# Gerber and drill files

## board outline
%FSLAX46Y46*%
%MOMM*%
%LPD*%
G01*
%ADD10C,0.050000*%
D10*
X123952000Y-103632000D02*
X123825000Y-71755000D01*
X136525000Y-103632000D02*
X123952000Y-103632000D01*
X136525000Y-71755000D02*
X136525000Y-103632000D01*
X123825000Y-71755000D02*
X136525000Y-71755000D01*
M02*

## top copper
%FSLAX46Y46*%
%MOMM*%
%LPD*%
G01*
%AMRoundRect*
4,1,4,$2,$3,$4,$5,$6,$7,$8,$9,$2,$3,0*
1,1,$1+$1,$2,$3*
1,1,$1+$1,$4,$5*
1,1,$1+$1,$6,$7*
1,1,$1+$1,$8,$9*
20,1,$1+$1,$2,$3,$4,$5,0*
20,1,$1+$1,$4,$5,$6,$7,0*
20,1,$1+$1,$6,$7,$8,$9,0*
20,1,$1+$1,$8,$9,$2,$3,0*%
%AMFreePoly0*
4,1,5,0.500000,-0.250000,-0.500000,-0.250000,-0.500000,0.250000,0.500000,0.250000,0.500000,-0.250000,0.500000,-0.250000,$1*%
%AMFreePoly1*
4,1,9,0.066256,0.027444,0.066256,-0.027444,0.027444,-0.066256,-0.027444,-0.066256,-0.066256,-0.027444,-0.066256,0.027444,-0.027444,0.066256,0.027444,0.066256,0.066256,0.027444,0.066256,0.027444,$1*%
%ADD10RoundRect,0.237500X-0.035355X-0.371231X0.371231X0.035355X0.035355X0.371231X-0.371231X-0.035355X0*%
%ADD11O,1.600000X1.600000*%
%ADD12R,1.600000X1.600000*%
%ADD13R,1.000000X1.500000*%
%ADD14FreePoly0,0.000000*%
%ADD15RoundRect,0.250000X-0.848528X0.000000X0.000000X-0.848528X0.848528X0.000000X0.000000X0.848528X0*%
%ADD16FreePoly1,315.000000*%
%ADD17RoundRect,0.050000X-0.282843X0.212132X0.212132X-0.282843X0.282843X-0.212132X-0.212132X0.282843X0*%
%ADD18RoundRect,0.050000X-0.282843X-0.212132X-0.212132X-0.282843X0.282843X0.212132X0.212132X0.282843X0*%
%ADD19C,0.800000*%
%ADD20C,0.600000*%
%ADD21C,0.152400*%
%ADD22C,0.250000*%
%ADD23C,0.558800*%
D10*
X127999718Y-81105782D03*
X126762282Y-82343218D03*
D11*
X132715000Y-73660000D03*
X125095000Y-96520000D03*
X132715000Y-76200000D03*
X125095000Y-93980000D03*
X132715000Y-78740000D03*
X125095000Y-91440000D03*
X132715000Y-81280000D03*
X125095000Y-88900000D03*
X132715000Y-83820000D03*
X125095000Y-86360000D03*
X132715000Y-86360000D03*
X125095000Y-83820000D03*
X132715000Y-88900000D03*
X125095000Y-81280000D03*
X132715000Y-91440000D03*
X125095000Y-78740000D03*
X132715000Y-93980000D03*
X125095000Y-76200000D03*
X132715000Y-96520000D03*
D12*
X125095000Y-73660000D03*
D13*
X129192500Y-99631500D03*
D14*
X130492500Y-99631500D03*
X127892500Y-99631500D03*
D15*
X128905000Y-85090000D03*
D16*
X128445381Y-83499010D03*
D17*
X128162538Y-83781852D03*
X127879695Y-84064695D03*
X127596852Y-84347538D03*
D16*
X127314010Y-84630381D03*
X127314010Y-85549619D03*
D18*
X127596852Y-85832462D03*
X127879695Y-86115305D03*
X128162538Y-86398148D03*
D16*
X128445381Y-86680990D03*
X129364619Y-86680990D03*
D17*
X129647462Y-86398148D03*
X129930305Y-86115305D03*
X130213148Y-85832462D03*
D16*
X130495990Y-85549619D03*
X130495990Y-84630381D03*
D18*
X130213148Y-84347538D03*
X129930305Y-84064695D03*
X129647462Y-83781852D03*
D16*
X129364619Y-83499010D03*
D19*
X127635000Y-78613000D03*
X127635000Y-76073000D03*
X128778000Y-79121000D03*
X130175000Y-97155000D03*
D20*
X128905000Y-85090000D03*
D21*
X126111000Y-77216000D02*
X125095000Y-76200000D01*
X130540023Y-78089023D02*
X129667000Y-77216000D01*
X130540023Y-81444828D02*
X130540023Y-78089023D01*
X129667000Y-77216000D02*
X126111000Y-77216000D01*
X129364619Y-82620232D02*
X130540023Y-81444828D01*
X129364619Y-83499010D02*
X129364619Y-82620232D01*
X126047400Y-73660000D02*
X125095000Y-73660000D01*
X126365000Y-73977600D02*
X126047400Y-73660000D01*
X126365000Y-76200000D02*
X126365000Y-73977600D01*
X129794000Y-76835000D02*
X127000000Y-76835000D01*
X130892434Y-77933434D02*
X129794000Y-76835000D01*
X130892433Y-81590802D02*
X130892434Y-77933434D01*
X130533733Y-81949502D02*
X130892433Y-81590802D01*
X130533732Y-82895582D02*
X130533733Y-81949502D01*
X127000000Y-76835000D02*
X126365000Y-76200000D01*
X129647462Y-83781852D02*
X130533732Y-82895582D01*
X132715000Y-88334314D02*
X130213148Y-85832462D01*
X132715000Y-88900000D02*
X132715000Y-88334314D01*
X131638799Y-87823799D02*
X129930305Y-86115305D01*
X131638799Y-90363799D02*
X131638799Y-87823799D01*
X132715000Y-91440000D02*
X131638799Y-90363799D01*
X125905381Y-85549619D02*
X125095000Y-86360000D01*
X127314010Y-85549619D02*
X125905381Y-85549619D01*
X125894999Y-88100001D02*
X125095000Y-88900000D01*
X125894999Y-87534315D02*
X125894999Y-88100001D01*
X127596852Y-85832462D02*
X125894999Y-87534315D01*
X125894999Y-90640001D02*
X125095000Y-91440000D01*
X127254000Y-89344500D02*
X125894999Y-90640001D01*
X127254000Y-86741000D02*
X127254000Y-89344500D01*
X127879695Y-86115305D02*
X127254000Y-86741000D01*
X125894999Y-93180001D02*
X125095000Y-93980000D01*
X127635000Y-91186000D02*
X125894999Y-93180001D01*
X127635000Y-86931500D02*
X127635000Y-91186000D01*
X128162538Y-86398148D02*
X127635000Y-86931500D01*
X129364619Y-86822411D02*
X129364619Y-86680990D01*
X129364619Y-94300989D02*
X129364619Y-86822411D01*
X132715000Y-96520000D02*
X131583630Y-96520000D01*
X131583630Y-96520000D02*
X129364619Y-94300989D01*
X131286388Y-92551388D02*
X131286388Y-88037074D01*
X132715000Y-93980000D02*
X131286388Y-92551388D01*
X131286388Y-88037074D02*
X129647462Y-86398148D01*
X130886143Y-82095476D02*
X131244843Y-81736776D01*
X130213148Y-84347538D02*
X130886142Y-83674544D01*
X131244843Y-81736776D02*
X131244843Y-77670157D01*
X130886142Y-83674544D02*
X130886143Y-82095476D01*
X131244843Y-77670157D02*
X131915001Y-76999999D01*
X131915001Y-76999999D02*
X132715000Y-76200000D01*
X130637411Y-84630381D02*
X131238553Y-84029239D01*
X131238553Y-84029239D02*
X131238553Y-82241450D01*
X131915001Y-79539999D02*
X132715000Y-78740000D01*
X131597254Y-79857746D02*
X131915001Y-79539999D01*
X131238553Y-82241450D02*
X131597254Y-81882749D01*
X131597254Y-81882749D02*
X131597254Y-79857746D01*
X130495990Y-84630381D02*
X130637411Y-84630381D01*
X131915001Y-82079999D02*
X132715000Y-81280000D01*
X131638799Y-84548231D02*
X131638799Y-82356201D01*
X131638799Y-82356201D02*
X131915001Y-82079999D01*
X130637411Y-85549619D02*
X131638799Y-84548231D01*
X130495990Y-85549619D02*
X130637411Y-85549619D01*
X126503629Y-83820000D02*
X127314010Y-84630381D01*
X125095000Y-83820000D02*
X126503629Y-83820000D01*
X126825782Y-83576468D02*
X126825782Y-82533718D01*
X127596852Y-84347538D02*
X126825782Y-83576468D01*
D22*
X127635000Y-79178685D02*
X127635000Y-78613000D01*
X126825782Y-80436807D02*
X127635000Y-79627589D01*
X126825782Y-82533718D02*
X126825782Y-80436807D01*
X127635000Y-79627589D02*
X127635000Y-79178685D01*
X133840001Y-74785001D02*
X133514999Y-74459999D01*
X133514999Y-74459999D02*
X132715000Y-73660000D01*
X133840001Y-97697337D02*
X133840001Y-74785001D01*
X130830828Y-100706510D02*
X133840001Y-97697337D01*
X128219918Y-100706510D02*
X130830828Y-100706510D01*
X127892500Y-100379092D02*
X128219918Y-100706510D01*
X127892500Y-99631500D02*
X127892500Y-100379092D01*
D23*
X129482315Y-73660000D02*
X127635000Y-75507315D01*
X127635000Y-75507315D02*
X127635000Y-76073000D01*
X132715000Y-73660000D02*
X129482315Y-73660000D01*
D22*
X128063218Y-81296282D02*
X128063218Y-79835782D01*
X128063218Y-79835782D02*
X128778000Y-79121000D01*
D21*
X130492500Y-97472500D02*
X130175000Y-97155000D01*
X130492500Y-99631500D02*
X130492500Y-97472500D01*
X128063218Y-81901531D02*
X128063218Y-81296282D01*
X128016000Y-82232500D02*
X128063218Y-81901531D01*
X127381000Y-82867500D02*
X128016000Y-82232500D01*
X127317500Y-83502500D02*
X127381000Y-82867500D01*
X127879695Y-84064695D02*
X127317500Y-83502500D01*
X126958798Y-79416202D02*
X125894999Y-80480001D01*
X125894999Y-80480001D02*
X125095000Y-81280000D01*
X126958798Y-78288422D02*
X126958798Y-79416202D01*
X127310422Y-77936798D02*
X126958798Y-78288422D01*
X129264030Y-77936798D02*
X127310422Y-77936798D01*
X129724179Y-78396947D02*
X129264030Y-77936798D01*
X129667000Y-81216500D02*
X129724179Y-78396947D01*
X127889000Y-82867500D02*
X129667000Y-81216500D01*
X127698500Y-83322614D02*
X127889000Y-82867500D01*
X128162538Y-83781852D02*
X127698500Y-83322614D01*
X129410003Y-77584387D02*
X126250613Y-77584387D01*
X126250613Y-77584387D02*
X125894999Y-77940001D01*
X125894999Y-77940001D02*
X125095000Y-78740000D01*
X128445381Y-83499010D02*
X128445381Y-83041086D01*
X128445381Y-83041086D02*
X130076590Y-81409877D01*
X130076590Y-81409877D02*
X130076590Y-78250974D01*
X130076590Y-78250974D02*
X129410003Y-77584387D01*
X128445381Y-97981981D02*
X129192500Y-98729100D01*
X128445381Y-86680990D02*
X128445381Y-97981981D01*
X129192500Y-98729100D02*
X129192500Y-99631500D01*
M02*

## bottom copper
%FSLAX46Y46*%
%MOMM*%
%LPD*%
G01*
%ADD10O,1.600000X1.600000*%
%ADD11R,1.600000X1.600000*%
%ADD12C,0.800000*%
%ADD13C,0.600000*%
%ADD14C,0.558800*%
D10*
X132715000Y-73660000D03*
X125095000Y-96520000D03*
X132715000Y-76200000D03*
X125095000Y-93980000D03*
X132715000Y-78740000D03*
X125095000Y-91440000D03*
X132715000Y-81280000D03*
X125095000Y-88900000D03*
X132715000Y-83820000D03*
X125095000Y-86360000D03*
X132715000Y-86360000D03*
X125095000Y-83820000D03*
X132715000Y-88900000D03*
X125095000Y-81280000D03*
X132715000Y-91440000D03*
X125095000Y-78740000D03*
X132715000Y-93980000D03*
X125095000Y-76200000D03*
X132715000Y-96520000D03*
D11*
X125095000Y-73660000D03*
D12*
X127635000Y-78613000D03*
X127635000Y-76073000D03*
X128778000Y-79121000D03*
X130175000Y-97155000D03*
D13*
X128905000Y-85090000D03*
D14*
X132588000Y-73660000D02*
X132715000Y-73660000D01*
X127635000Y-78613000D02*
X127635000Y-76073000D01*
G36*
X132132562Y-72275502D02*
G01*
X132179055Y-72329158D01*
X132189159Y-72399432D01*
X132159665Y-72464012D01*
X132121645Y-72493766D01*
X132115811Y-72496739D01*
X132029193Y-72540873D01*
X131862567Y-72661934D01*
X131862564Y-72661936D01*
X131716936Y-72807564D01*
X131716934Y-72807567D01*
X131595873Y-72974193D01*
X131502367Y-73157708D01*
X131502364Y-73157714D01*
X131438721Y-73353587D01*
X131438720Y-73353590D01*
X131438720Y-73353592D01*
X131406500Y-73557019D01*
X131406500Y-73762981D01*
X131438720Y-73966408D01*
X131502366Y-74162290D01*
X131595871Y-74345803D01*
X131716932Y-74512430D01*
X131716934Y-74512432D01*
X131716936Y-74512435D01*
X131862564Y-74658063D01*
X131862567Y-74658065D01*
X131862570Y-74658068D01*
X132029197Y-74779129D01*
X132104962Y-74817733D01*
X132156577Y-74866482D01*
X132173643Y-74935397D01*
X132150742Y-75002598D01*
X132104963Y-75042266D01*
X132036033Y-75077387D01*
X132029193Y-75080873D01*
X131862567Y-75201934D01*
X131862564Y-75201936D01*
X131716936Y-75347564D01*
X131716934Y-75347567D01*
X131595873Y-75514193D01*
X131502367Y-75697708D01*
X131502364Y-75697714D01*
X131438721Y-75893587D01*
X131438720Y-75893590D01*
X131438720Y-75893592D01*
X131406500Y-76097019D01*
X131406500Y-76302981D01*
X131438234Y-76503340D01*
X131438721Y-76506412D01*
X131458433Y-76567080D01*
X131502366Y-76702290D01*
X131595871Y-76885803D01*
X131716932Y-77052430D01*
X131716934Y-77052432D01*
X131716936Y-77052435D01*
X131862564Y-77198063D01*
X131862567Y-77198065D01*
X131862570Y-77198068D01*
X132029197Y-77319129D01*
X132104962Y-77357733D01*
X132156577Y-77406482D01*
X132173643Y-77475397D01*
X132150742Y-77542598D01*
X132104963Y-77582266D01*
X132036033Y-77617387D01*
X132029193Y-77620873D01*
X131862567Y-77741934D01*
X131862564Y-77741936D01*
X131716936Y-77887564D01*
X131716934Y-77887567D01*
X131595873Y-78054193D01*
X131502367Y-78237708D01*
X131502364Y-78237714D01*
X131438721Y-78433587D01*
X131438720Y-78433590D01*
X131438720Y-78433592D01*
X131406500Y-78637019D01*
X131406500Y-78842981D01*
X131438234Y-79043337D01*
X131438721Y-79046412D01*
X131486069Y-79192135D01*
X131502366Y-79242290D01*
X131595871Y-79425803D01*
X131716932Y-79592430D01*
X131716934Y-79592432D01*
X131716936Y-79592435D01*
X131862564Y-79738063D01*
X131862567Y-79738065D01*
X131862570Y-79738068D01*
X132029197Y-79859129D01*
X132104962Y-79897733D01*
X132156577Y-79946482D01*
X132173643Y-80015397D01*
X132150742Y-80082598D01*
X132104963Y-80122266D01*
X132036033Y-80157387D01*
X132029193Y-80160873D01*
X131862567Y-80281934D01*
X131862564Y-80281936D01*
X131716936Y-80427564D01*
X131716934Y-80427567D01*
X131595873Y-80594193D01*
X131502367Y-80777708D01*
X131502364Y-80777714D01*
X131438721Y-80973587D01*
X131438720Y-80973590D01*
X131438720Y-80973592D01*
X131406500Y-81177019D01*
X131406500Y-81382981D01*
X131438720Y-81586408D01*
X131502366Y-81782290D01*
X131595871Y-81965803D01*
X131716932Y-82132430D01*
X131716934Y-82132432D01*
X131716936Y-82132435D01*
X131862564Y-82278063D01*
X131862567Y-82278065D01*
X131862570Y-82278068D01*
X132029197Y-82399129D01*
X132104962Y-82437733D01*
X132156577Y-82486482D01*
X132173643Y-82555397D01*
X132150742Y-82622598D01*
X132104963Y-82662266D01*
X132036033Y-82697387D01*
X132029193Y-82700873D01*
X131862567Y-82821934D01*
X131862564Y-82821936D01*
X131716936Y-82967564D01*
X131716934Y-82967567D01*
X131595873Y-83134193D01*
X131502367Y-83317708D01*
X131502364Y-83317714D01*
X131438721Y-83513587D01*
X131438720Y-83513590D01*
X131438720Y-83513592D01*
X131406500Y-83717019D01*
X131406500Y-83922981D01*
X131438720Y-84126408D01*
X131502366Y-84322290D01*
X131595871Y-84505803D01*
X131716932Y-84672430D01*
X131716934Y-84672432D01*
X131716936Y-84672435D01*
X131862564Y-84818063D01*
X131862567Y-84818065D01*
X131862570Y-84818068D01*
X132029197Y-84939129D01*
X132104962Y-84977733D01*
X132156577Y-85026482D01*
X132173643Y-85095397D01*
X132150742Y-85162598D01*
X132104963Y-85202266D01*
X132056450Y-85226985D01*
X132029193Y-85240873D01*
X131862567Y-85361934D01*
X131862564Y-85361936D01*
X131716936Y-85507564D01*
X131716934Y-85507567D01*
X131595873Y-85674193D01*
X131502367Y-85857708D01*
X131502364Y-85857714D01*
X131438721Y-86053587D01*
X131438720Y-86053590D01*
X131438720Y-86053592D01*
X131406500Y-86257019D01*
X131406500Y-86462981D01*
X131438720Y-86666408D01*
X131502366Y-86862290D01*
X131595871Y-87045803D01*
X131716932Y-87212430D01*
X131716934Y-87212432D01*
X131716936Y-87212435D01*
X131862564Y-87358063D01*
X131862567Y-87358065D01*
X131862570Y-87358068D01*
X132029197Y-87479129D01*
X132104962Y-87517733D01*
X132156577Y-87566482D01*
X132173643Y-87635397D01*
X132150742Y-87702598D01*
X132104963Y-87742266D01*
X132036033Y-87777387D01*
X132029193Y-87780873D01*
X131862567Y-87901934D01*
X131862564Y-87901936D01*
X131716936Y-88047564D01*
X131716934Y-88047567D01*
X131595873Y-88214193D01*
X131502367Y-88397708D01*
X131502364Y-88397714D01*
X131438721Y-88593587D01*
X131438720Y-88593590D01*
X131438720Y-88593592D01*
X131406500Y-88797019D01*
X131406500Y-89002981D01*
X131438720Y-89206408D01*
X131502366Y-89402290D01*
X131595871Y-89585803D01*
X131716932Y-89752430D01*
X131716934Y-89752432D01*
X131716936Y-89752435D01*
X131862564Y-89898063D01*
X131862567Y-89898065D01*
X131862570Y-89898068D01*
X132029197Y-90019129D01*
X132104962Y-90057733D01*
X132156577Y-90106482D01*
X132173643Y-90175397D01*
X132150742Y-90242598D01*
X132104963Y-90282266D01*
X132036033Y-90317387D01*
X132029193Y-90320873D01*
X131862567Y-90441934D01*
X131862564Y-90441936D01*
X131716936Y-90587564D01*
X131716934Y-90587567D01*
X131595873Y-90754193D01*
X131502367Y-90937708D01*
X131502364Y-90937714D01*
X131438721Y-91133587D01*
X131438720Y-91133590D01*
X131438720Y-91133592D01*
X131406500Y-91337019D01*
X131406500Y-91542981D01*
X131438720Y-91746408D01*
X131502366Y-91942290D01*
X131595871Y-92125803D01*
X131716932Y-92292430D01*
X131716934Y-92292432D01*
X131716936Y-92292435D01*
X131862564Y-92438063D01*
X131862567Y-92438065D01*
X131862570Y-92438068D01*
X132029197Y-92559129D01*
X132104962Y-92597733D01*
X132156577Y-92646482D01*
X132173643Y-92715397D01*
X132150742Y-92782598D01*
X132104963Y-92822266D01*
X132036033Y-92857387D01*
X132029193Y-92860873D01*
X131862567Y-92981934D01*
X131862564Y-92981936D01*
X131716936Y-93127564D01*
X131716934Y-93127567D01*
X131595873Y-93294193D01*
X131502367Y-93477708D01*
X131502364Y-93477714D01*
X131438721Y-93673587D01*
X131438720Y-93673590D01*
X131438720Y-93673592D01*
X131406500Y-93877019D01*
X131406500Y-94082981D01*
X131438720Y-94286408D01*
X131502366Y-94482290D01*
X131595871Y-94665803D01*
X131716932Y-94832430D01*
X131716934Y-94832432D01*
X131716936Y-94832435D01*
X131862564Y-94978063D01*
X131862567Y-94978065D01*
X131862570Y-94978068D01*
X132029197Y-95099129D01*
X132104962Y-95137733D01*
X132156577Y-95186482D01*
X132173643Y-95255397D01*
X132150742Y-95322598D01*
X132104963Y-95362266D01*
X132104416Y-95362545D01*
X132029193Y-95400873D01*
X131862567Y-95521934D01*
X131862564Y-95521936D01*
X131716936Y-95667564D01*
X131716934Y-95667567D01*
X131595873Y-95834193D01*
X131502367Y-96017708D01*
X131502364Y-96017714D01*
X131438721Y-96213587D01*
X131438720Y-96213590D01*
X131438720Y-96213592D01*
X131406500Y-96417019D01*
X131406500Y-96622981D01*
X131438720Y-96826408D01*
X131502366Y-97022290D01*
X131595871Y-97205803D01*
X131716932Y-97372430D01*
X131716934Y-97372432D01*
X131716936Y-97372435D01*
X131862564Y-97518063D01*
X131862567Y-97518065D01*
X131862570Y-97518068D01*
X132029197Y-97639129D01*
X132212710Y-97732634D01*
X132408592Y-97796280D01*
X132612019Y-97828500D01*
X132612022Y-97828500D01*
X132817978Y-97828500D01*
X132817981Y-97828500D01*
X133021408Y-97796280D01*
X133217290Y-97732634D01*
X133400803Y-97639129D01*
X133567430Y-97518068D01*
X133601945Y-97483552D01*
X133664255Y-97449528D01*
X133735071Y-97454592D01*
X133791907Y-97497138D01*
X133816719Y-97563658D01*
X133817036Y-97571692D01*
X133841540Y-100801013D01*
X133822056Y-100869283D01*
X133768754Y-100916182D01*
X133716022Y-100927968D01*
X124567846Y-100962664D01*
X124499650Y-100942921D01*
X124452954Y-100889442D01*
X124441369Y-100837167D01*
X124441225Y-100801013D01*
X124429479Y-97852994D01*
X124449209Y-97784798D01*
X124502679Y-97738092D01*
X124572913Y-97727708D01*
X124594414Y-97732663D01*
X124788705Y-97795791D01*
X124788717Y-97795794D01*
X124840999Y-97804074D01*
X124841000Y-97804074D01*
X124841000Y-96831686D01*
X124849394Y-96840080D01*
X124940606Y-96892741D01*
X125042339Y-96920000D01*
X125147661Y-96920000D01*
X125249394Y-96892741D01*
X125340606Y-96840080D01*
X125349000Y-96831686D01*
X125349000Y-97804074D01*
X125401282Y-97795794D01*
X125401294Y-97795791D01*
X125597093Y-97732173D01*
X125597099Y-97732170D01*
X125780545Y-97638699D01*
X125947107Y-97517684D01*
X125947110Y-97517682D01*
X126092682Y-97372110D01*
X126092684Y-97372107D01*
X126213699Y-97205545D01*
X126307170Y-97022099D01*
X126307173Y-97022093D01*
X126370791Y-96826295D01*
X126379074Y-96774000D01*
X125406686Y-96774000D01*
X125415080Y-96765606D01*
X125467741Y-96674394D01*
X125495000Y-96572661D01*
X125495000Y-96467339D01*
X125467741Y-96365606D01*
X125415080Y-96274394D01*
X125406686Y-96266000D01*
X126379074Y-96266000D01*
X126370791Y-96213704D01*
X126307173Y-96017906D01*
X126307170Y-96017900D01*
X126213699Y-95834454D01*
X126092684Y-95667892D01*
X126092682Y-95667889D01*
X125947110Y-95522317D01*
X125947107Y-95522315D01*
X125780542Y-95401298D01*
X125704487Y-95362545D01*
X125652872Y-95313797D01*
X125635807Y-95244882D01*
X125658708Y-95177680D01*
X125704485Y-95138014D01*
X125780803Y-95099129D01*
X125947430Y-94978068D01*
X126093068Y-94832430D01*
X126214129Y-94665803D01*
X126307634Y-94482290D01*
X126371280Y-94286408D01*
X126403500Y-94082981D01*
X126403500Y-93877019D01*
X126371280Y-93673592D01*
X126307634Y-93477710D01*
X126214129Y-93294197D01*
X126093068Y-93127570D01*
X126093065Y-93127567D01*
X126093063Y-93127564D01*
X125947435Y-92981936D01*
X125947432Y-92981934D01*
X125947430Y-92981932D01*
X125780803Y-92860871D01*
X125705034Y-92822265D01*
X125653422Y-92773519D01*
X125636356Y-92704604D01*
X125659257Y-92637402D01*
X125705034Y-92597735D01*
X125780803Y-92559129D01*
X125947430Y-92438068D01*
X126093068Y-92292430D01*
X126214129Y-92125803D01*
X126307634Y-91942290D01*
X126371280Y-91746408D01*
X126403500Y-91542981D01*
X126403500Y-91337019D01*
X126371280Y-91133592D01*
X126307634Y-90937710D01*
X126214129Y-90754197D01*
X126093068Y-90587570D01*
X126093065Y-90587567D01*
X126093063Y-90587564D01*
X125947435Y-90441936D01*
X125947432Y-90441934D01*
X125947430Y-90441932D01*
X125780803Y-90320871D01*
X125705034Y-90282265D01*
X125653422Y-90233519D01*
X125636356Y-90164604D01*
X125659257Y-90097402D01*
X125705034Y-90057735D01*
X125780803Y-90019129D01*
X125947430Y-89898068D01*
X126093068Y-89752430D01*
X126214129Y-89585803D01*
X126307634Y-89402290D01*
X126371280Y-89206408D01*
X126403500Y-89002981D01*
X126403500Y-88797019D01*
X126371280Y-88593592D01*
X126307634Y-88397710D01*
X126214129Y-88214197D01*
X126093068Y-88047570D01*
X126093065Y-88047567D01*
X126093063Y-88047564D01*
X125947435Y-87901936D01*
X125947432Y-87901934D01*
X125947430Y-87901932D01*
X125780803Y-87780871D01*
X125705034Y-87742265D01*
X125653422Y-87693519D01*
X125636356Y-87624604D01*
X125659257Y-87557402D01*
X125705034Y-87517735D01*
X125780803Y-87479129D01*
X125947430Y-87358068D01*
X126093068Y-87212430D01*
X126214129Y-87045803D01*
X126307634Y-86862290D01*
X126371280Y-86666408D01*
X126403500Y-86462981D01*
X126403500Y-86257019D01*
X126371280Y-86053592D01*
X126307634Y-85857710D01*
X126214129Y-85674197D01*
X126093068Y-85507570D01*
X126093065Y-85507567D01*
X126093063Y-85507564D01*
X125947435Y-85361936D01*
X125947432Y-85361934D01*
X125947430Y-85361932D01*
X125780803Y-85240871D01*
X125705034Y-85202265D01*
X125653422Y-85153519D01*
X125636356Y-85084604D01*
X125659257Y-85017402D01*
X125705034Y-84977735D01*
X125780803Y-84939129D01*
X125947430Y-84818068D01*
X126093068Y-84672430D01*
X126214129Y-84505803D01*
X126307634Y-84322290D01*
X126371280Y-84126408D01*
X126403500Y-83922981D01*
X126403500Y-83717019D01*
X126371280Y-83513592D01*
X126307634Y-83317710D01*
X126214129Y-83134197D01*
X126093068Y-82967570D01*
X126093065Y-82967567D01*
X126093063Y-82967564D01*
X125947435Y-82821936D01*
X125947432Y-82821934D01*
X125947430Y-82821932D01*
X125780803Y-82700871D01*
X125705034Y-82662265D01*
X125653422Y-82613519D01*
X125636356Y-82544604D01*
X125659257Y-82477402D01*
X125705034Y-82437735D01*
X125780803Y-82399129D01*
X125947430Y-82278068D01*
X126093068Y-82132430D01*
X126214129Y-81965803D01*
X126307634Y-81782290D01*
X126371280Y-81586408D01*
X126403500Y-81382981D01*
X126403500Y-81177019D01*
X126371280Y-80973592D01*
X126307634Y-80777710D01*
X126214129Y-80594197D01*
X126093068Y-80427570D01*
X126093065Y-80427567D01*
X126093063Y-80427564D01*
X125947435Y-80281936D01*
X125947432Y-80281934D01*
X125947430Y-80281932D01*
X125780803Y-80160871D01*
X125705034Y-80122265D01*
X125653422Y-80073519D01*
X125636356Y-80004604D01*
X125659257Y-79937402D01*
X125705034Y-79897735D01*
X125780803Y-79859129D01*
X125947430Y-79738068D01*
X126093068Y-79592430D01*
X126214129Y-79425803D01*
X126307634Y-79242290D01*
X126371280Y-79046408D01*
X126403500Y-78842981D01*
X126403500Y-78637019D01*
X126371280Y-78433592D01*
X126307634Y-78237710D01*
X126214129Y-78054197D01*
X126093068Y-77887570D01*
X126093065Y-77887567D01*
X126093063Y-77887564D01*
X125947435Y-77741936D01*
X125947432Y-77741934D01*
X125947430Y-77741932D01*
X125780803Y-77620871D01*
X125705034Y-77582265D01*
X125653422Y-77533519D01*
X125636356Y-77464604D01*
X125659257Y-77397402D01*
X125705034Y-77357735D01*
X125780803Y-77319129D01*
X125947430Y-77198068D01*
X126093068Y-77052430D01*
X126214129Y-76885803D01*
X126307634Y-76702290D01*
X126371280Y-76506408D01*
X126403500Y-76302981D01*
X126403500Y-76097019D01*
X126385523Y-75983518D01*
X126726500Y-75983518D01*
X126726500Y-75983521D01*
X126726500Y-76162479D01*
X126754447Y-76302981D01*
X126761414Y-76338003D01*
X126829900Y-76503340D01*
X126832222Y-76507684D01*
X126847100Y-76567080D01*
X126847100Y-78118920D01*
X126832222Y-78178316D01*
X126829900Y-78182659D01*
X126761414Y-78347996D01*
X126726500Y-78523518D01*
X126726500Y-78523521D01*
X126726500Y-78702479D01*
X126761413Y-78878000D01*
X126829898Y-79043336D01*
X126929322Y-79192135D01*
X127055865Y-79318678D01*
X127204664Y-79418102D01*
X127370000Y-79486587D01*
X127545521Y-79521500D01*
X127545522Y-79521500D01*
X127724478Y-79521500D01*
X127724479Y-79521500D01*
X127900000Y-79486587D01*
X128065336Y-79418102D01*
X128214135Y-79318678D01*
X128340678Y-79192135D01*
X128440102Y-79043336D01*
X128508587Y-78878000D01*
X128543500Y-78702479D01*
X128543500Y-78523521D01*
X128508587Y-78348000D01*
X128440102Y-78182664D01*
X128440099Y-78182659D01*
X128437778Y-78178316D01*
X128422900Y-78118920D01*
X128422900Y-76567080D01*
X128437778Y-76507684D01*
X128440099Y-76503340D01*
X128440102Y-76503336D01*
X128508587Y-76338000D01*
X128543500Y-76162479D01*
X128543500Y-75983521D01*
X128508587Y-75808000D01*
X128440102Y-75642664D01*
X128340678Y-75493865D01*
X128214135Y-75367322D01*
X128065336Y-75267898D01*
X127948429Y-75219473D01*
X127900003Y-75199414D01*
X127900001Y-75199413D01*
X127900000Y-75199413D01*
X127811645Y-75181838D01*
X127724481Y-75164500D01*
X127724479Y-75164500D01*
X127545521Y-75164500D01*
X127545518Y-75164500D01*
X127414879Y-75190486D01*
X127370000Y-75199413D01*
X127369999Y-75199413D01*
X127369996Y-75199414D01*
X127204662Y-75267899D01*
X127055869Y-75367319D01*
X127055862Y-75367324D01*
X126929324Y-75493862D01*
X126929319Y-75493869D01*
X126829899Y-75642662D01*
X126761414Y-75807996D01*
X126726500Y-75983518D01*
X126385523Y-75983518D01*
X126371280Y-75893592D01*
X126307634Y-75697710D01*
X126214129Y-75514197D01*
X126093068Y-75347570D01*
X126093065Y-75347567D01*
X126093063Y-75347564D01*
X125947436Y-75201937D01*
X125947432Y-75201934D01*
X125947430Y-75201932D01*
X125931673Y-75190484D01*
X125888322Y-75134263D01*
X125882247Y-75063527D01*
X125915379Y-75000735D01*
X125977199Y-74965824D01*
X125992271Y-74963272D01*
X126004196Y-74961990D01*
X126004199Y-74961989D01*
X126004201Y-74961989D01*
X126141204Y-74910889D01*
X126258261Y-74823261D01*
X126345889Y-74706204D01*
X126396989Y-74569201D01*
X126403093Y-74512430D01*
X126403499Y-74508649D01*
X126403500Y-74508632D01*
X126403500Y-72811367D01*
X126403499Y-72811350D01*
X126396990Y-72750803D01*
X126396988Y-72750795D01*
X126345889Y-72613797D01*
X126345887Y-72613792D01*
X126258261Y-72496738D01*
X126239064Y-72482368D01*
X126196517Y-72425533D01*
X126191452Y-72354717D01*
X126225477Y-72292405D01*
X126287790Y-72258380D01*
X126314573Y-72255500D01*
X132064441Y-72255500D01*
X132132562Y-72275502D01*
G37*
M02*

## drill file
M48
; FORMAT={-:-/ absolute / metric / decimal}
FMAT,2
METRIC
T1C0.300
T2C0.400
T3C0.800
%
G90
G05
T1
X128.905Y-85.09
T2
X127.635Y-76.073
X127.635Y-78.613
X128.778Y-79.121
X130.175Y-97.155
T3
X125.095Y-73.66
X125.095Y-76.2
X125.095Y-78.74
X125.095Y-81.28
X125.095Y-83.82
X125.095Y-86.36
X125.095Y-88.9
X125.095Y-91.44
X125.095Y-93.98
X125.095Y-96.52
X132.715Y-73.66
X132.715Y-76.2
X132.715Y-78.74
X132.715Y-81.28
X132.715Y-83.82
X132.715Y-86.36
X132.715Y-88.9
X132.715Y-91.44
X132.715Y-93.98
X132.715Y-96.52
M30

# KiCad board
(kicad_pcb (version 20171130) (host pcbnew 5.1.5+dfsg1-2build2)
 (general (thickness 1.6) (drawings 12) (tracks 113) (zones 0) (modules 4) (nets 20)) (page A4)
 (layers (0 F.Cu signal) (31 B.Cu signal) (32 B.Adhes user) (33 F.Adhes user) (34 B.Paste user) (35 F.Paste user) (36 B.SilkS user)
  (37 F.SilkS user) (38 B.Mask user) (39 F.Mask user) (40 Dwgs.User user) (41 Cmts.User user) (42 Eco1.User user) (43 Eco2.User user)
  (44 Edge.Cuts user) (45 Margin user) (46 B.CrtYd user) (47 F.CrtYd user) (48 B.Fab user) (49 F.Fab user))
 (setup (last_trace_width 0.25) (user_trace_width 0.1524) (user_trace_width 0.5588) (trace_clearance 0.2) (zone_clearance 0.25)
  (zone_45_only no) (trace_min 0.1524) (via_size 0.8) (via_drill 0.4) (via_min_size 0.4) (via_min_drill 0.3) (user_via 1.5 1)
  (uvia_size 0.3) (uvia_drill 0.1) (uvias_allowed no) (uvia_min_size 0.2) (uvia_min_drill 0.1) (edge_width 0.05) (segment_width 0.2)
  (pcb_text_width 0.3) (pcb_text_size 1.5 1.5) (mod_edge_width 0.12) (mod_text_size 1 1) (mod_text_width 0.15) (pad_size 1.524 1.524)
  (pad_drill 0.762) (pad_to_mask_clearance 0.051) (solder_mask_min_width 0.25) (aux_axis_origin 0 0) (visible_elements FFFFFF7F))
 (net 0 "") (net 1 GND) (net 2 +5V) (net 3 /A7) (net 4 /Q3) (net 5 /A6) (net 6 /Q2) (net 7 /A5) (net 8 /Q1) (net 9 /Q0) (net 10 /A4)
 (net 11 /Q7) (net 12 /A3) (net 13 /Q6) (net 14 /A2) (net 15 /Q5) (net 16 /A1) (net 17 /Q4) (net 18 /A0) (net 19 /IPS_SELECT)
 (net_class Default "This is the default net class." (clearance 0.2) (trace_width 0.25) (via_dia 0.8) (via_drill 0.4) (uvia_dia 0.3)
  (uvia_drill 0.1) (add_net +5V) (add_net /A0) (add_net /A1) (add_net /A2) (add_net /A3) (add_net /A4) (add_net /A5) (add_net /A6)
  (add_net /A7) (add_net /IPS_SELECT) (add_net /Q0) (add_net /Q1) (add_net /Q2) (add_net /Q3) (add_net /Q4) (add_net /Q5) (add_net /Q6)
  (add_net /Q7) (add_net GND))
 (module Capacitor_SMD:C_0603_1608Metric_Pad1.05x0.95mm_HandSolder (layer F.Cu) (at 127.381 81.7245 45)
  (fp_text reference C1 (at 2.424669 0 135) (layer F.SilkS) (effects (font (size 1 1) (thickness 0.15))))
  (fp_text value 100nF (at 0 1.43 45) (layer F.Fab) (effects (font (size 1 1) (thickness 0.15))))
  (pad 2 smd roundrect (at 0.875 0 45) (size 1.05 0.95) (layers F.Cu F.Paste F.Mask) (roundrect_rratio 0.25) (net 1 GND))
  (pad 1 smd roundrect (at -0.875 0 45) (size 1.05 0.95) (layers F.Cu F.Paste F.Mask) (roundrect_rratio 0.25) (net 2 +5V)))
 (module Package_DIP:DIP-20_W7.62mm (layer F.Cu) (at 125.095 73.66)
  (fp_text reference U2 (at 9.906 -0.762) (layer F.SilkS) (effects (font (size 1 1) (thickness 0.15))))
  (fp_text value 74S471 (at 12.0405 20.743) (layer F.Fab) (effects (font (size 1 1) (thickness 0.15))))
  (pad 20 thru_hole oval (at 7.62 0) (size 1.6 1.6) (drill 0.8) (layers *.Cu *.Mask) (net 2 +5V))
  (pad 10 thru_hole oval (at 0 22.86) (size 1.6 1.6) (drill 0.8) (layers *.Cu *.Mask) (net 1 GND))
  (pad 19 thru_hole oval (at 7.62 2.54) (size 1.6 1.6) (drill 0.8) (layers *.Cu *.Mask) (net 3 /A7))
  (pad 9 thru_hole oval (at 0 20.32) (size 1.6 1.6) (drill 0.8) (layers *.Cu *.Mask) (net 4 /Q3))
  (pad 18 thru_hole oval (at 7.62 5.08) (size 1.6 1.6) (drill 0.8) (layers *.Cu *.Mask) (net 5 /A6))
  (pad 8 thru_hole oval (at 0 17.78) (size 1.6 1.6) (drill 0.8) (layers *.Cu *.Mask) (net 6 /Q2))
  (pad 17 thru_hole oval (at 7.62 7.62) (size 1.6 1.6) (drill 0.8) (layers *.Cu *.Mask) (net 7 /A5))
  (pad 7 thru_hole oval (at 0 15.24) (size 1.6 1.6) (drill 0.8) (layers *.Cu *.Mask) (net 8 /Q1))
  (pad 16 thru_hole oval (at 7.62 10.16) (size 1.6 1.6) (drill 0.8) (layers *.Cu *.Mask))
  (pad 6 thru_hole oval (at 0 12.7) (size 1.6 1.6) (drill 0.8) (layers *.Cu *.Mask) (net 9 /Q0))
  (pad 15 thru_hole oval (at 7.62 12.7) (size 1.6 1.6) (drill 0.8) (layers *.Cu *.Mask))
  (pad 5 thru_hole oval (at 0 10.16) (size 1.6 1.6) (drill 0.8) (layers *.Cu *.Mask) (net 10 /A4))
  (pad 14 thru_hole oval (at 7.62 15.24) (size 1.6 1.6) (drill 0.8) (layers *.Cu *.Mask) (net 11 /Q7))
  (pad 4 thru_hole oval (at 0 7.62) (size 1.6 1.6) (drill 0.8) (layers *.Cu *.Mask) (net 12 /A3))
  (pad 13 thru_hole oval (at 7.62 17.78) (size 1.6 1.6) (drill 0.8) (layers *.Cu *.Mask) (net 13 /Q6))
  (pad 3 thru_hole oval (at 0 5.08) (size 1.6 1.6) (drill 0.8) (layers *.Cu *.Mask) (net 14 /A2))
  (pad 12 thru_hole oval (at 7.62 20.32) (size 1.6 1.6) (drill 0.8) (layers *.Cu *.Mask) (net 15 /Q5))
  (pad 2 thru_hole oval (at 0 2.54) (size 1.6 1.6) (drill 0.8) (layers *.Cu *.Mask) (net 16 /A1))
  (pad 11 thru_hole oval (at 7.62 22.86) (size 1.6 1.6) (drill 0.8) (layers *.Cu *.Mask) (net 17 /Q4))
  (pad 1 thru_hole rect (at 0 0) (size 1.6 1.6) (drill 0.8) (layers *.Cu *.Mask) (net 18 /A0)))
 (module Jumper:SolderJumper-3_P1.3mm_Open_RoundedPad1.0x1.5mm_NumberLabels (layer F.Cu) (at 129.1925 99.6315)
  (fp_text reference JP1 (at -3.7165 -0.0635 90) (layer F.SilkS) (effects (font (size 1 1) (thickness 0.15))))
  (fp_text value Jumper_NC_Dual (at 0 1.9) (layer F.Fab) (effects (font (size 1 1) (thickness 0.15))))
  (pad 2 smd rect (at 0 0) (size 1 1.5) (layers F.Cu F.Mask) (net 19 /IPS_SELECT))
  (pad 3 smd custom (at 1.3 0) (size 1 0.5) (layers F.Cu F.Mask) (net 1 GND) (zone_connect 2) (options (clearance outline) (anchor rect))
   (primitives))
  (pad 1 smd custom (at -1.3 0) (size 1 0.5) (layers F.Cu F.Mask) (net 2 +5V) (zone_connect 2) (options (clearance outline) (anchor rect))
   (primitives)))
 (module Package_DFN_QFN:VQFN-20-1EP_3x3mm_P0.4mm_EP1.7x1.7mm (layer F.Cu) (at 128.905 85.09 315)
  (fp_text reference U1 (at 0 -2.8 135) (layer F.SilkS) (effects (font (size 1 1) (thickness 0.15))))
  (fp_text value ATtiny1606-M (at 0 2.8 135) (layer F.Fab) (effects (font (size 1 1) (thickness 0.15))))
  (pad 21 smd roundrect (at 0 0 315) (size 1.7 1.7) (layers F.Cu F.Mask) (roundrect_rratio 0.147059) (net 1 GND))
  (pad "" smd roundrect (at -0.425 -0.425 315) (size 0.69 0.69) (layers F.Paste) (roundrect_rratio 0.25))
  (pad "" smd roundrect (at -0.425 0.425 315) (size 0.69 0.69) (layers F.Paste) (roundrect_rratio 0.25))
  (pad "" smd roundrect (at 0.425 -0.425 315) (size 0.69 0.69) (layers F.Paste) (roundrect_rratio 0.25))
  (pad "" smd roundrect (at 0.425 0.425 315) (size 0.69 0.69) (layers F.Paste) (roundrect_rratio 0.25))
  (pad 1 smd custom (at -1.45 -0.8 315) (size 0.143431 0.143431) (layers F.Cu F.Paste F.Mask) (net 14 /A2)
   (options (clearance outline) (anchor circle)) (primitives))
  (pad 2 smd roundrect (at -1.45 -0.4 315) (size 0.8 0.2) (layers F.Cu F.Paste F.Mask) (roundrect_rratio 0.25) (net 12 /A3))
  (pad 3 smd roundrect (at -1.45 0 315) (size 0.8 0.2) (layers F.Cu F.Paste F.Mask) (roundrect_rratio 0.25) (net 1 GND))
  (pad 4 smd roundrect (at -1.45 0.4 315) (size 0.8 0.2) (layers F.Cu F.Paste F.Mask) (roundrect_rratio 0.25) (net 2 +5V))
  (pad 5 smd custom (at -1.45 0.8 315) (size 0.143431 0.143431) (layers F.Cu F.Paste F.Mask) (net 10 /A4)
   (options (clearance outline) (anchor circle)) (primitives))
  (pad 6 smd custom (at -0.8 1.45 315) (size 0.143431 0.143431) (layers F.Cu F.Paste F.Mask) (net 9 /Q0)
   (options (clearance outline) (anchor circle)) (primitives))
  (pad 7 smd roundrect (at -0.4 1.45 315) (size 0.2 0.8) (layers F.Cu F.Paste F.Mask) (roundrect_rratio 0.25) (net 8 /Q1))
  (pad 8 smd roundrect (at 0 1.45 315) (size 0.2 0.8) (layers F.Cu F.Paste F.Mask) (roundrect_rratio 0.25) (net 6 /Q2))
  (pad 9 smd roundrect (at 0.4 1.45 315) (size 0.2 0.8) (layers F.Cu F.Paste F.Mask) (roundrect_rratio 0.25) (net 4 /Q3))
  (pad 10 smd custom (at 0.8 1.45 315) (size 0.143431 0.143431) (layers F.Cu F.Paste F.Mask) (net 19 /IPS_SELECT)
   (options (clearance outline) (anchor circle)) (primitives))
  (pad 11 smd custom (at 1.45 0.8 315) (size 0.143431 0.143431) (layers F.Cu F.Paste F.Mask) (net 17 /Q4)
   (options (clearance outline) (anchor circle)) (primitives))
  (pad 12 smd roundrect (at 1.45 0.4 315) (size 0.8 0.2) (layers F.Cu F.Paste F.Mask) (roundrect_rratio 0.25) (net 15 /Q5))
  (pad 13 smd roundrect (at 1.45 0 315) (size 0.8 0.2) (layers F.Cu F.Paste F.Mask) (roundrect_rratio 0.25) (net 13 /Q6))
  (pad 14 smd roundrect (at 1.45 -0.4 315) (size 0.8 0.2) (layers F.Cu F.Paste F.Mask) (roundrect_rratio 0.25) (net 11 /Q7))
  (pad 15 smd custom (at 1.45 -0.8 315) (size 0.143431 0.143431) (layers F.Cu F.Paste F.Mask) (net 7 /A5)
   (options (clearance outline) (anchor circle)) (primitives))
  (pad 16 smd custom (at 0.8 -1.45 315) (size 0.143431 0.143431) (layers F.Cu F.Paste F.Mask) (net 5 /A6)
   (options (clearance outline) (anchor circle)) (primitives))
  (pad 17 smd roundrect (at 0.4 -1.45 315) (size 0.2 0.8) (layers F.Cu F.Paste F.Mask) (roundrect_rratio 0.25) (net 3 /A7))
  (pad 18 smd roundrect (at 0 -1.45 315) (size 0.2 0.8) (layers F.Cu F.Paste F.Mask) (roundrect_rratio 0.25))
  (pad 19 smd roundrect (at -0.4 -1.45 315) (size 0.2 0.8) (layers F.Cu F.Paste F.Mask) (roundrect_rratio 0.25) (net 18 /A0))
  (pad 20 smd custom (at -0.8 -1.45 315) (size 0.143431 0.143431) (layers F.Cu F.Paste F.Mask) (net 16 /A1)
   (options (clearance outline) (anchor circle)) (primitives)))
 (gr_line (start 123.952 103.632) (end 123.825 71.755) (layer Edge.Cuts) (width 0.05))
 (gr_line (start 136.525 103.632) (end 123.952 103.632) (layer Edge.Cuts) (width 0.05))
 (gr_line (start 136.525 71.755) (end 136.525 103.632) (layer Edge.Cuts) (width 0.05))
 (gr_line (start 123.825 71.755) (end 136.525 71.755) (layer Edge.Cuts) (width 0.05))
 (segment (start 126.111 77.216) (end 125.095 76.2) (width 0.1524) (layer F.Cu) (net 16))
 (segment (start 130.540023 78.089023) (end 129.667 77.216) (width 0.1524) (layer F.Cu) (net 16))
 (segment (start 130.540023 81.444828) (end 130.540023 78.089023) (width 0.1524) (layer F.Cu) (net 16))
 (segment (start 129.667 77.216) (end 126.111 77.216) (width 0.1524) (layer F.Cu) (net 16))
 (segment (start 129.364619 82.620232) (end 130.540023 81.444828) (width 0.1524) (layer F.Cu) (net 16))
 (segment (start 129.364619 83.49901) (end 129.364619 82.620232) (width 0.1524) (layer F.Cu) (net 16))
 (segment (start 126.0474 73.66) (end 125.095 73.66) (width 0.1524) (layer F.Cu) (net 18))
 (segment (start 126.365 73.9776) (end 126.0474 73.66) (width 0.1524) (layer F.Cu) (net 18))
 (segment (start 126.365 76.2) (end 126.365 73.9776) (width 0.1524) (layer F.Cu) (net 18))
 (segment (start 129.794 76.835) (end 127 76.835) (width 0.1524) (layer F.Cu) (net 18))
 (segment (start 130.892434 77.933434) (end 129.794 76.835) (width 0.1524) (layer F.Cu) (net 18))
 (segment (start 130.892433 81.590802) (end 130.892434 77.933434) (width 0.1524) (layer F.Cu) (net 18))
 (segment (start 130.533733 81.949502) (end 130.892433 81.590802) (width 0.1524) (layer F.Cu) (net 18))
 (segment (start 130.533732 82.895582) (end 130.533733 81.949502) (width 0.1524) (layer F.Cu) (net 18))
 (segment (start 127 76.835) (end 126.365 76.2) (width 0.1524) (layer F.Cu) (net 18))
 (segment (start 129.647462 83.781852) (end 130.533732 82.895582) (width 0.1524) (layer F.Cu) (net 18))
 (segment (start 132.715 88.334314) (end 130.213148 85.832462) (width 0.1524) (layer F.Cu) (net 11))
 (segment (start 132.715 88.9) (end 132.715 88.334314) (width 0.1524) (layer F.Cu) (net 11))
 (segment (start 131.638799 87.823799) (end 129.930305 86.115305) (width 0.1524) (layer F.Cu) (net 13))
 (segment (start 131.638799 90.363799) (end 131.638799 87.823799) (width 0.1524) (layer F.Cu) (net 13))
 (segment (start 132.715 91.44) (end 131.638799 90.363799) (width 0.1524) (layer F.Cu) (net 13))
 (segment (start 125.905381 85.549619) (end 125.095 86.36) (width 0.1524) (layer F.Cu) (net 9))
 (segment (start 127.31401 85.549619) (end 125.905381 85.549619) (width 0.1524) (layer F.Cu) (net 9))
 (segment (start 125.894999 88.100001) (end 125.095 88.9) (width 0.1524) (layer F.Cu) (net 8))
 (segment (start 125.894999 87.534315) (end 125.894999 88.100001) (width 0.1524) (layer F.Cu) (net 8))
 (segment (start 127.596852 85.832462) (end 125.894999 87.534315) (width 0.1524) (layer F.Cu) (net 8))
 (segment (start 125.894999 90.640001) (end 125.095 91.44) (width 0.1524) (layer F.Cu) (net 6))
 (segment (start 127.254 89.3445) (end 125.894999 90.640001) (width 0.1524) (layer F.Cu) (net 6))
 (segment (start 127.254 86.741) (end 127.254 89.3445) (width 0.1524) (layer F.Cu) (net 6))
 (segment (start 127.879695 86.115305) (end 127.254 86.741) (width 0.1524) (layer F.Cu) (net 6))
 (segment (start 125.894999 93.180001) (end 125.095 93.98) (width 0.1524) (layer F.Cu) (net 4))
 (segment (start 127.635 91.186) (end 125.894999 93.180001) (width 0.1524) (layer F.Cu) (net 4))
 (segment (start 127.635 86.9315) (end 127.635 91.186) (width 0.1524) (layer F.Cu) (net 4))
 (segment (start 128.162538 86.398148) (end 127.635 86.9315) (width 0.1524) (layer F.Cu) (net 4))
 (segment (start 129.364619 86.822411) (end 129.364619 86.68099) (width 0.1524) (layer F.Cu) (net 17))
 (segment (start 129.364619 94.300989) (end 129.364619 86.822411) (width 0.1524) (layer F.Cu) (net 17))
 (segment (start 132.715 96.52) (end 131.58363 96.52) (width 0.1524) (layer F.Cu) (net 17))
 (segment (start 131.58363 96.52) (end 129.364619 94.300989) (width 0.1524) (layer F.Cu) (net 17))
 (segment (start 131.286388 92.551388) (end 131.286388 88.037074) (width 0.1524) (layer F.Cu) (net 15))
 (segment (start 132.715 93.98) (end 131.286388 92.551388) (width 0.1524) (layer F.Cu) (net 15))
 (segment (start 131.286388 88.037074) (end 129.647462 86.398148) (width 0.1524) (layer F.Cu) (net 15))
 (segment (start 130.886143 82.095476) (end 131.244843 81.736776) (width 0.1524) (layer F.Cu) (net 3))
 (segment (start 130.213148 84.347538) (end 130.886142 83.674544) (width 0.1524) (layer F.Cu) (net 3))
 (segment (start 131.244843 81.736776) (end 131.244843 77.670157) (width 0.1524) (layer F.Cu) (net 3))
 (segment (start 130.886142 83.674544) (end 130.886143 82.095476) (width 0.1524) (layer F.Cu) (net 3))
 (segment (start 131.244843 77.670157) (end 131.915001 76.999999) (width 0.1524) (layer F.Cu) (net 3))
 (segment (start 131.915001 76.999999) (end 132.715 76.2) (width 0.1524) (layer F.Cu) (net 3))
 (segment (start 130.637411 84.630381) (end 131.238553 84.029239) (width 0.1524) (layer F.Cu) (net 5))
 (segment (start 131.238553 84.029239) (end 131.238553 82.24145) (width 0.1524) (layer F.Cu) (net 5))
 (segment (start 131.915001 79.539999) (end 132.715 78.74) (width 0.1524) (layer F.Cu) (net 5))
 (segment (start 131.597254 79.857746) (end 131.915001 79.539999) (width 0.1524) (layer F.Cu) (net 5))
 (segment (start 131.238553 82.24145) (end 131.597254 81.882749) (width 0.1524) (layer F.Cu) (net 5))
 (segment (start 131.597254 81.882749) (end 131.597254 79.857746) (width 0.1524) (layer F.Cu) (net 5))
 (segment (start 130.49599 84.630381) (end 130.637411 84.630381) (width 0.1524) (layer F.Cu) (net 5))
 (segment (start 131.915001 82.079999) (end 132.715 81.28) (width 0.1524) (layer F.Cu) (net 7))
 (segment (start 131.638799 84.548231) (end 131.638799 82.356201) (width 0.1524) (layer F.Cu) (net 7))
 (segment (start 131.638799 82.356201) (end 131.915001 82.079999) (width 0.1524) (layer F.Cu) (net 7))
 (segment (start 130.637411 85.549619) (end 131.638799 84.548231) (width 0.1524) (layer F.Cu) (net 7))
 (segment (start 130.49599 85.549619) (end 130.637411 85.549619) (width 0.1524) (layer F.Cu) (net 7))
 (segment (start 126.503629 83.82) (end 127.31401 84.630381) (width 0.1524) (layer F.Cu) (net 10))
 (segment (start 125.095 83.82) (end 126.503629 83.82) (width 0.1524) (layer F.Cu) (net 10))
 (segment (start 126.825782 83.576468) (end 126.825782 82.533718) (width 0.1524) (layer F.Cu) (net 2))
 (segment (start 127.596852 84.347538) (end 126.825782 83.576468) (width 0.1524) (layer F.Cu) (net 2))
 (via (at 127.635 78.613) (size 0.8) (drill 0.4) (layers F.Cu B.Cu) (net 2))
 (segment (start 127.635 79.178685) (end 127.635 78.613) (width 0.25) (layer F.Cu) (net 2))
 (segment (start 126.825782 80.436807) (end 127.635 79.627589) (width 0.25) (layer F.Cu) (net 2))
 (segment (start 126.825782 82.533718) (end 126.825782 80.436807) (width 0.25) (layer F.Cu) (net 2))
 (segment (start 127.635 79.627589) (end 127.635 79.178685) (width 0.25) (layer F.Cu) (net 2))
 (segment (start 132.588 73.66) (end 132.715 73.66) (width 0.5588) (layer B.Cu) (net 2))
 (segment (start 133.840001 74.785001) (end 133.514999 74.459999) (width 0.25) (layer F.Cu) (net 2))
 (segment (start 133.514999 74.459999) (end 132.715 73.66) (width 0.25) (layer F.Cu) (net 2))
 (segment (start 133.840001 97.697337) (end 133.840001 74.785001) (width 0.25) (layer F.Cu) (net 2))
 (segment (start 130.830828 100.70651) (end 133.840001 97.697337) (width 0.25) (layer F.Cu) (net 2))
 (segment (start 128.219918 100.70651) (end 130.830828 100.70651) (width 0.25) (layer F.Cu) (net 2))
 (segment (start 127.8925 100.379092) (end 128.219918 100.70651) (width 0.25) (layer F.Cu) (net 2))
 (segment (start 127.8925 99.6315) (end 127.8925 100.379092) (width 0.25) (layer F.Cu) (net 2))
 (via (at 127.635 76.073) (size 0.8) (drill 0.4) (layers F.Cu B.Cu) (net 2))
 (segment (start 129.482315 73.66) (end 127.635 75.507315) (width 0.5588) (layer F.Cu) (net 2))
 (segment (start 127.635 75.507315) (end 127.635 76.073) (width 0.5588) (layer F.Cu) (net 2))
 (segment (start 132.715 73.66) (end 129.482315 73.66) (width 0.5588) (layer F.Cu) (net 2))
 (segment (start 127.635 78.613) (end 127.635 76.073) (width 0.5588) (layer B.Cu) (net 2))
 (via (at 128.778 79.121) (size 0.8) (drill 0.4) (layers F.Cu B.Cu) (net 1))
 (segment (start 128.063218 81.296282) (end 128.063218 79.835782) (width 0.25) (layer F.Cu) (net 1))
 (segment (start 128.063218 79.835782) (end 128.778 79.121) (width 0.25) (layer F.Cu) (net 1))
 (segment (start 130.4925 97.4725) (end 130.175 97.155) (width 0.1524) (layer F.Cu) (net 1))
 (via (at 130.175 97.155) (size 0.8) (drill 0.4) (layers F.Cu B.Cu) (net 1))
 (segment (start 130.4925 99.6315) (end 130.4925 97.4725) (width 0.1524) (layer F.Cu) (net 1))
 (via (at 128.905 85.09) (size 0.6) (drill 0.3) (layers F.Cu B.Cu) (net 1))
 (segment (start 128.063218 81.901531) (end 128.063218 81.296282) (width 0.1524) (layer F.Cu) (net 1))
 (segment (start 128.016 82.2325) (end 128.063218 81.901531) (width 0.1524) (layer F.Cu) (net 1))
 (segment (start 127.381 82.8675) (end 128.016 82.2325) (width 0.1524) (layer F.Cu) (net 1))
 (segment (start 127.3175 83.5025) (end 127.381 82.8675) (width 0.1524) (layer F.Cu) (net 1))
 (segment (start 127.879695 84.064695) (end 127.3175 83.5025) (width 0.1524) (layer F.Cu) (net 1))
 (segment (start 126.958798 79.416202) (end 125.894999 80.480001) (width 0.1524) (layer F.Cu) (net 12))
 (segment (start 125.894999 80.480001) (end 125.095 81.28) (width 0.1524) (layer F.Cu) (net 12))
 (segment (start 126.958798 78.288422) (end 126.958798 79.416202) (width 0.1524) (layer F.Cu) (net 12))
 (segment (start 127.310422 77.936798) (end 126.958798 78.288422) (width 0.1524) (layer F.Cu) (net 12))
 (segment (start 129.26403 77.936798) (end 127.310422 77.936798) (width 0.1524) (layer F.Cu) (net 12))
 (segment (start 129.724179 78.396947) (end 129.26403 77.936798) (width 0.1524) (layer F.Cu) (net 12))
 (segment (start 129.667 81.2165) (end 129.724179 78.396947) (width 0.1524) (layer F.Cu) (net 12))
 (segment (start 127.889 82.8675) (end 129.667 81.2165) (width 0.1524) (layer F.Cu) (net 12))
 (segment (start 127.6985 83.322614) (end 127.889 82.8675) (width 0.1524) (layer F.Cu) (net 12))
 (segment (start 128.162538 83.781852) (end 127.6985 83.322614) (width 0.1524) (layer F.Cu) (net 12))
 (segment (start 129.410003 77.584387) (end 126.250613 77.584387) (width 0.1524) (layer F.Cu) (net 14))
 (segment (start 126.250613 77.584387) (end 125.894999 77.940001) (width 0.1524) (layer F.Cu) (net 14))
 (segment (start 125.894999 77.940001) (end 125.095 78.74) (width 0.1524) (layer F.Cu) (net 14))
 (segment (start 128.445381 83.49901) (end 128.445381 83.041086) (width 0.1524) (layer F.Cu) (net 14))
 (segment (start 128.445381 83.041086) (end 130.07659 81.409877) (width 0.1524) (layer F.Cu) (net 14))
 (segment (start 130.07659 81.409877) (end 130.07659 78.250974) (width 0.1524) (layer F.Cu) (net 14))
 (segment (start 130.07659 78.250974) (end 129.410003 77.584387) (width 0.1524) (layer F.Cu) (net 14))
 (segment (start 128.445381 97.981981) (end 129.1925 98.7291) (width 0.1524) (layer F.Cu) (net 19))
 (segment (start 128.445381 86.68099) (end 128.445381 97.981981) (width 0.1524) (layer F.Cu) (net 19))
 (segment (start 129.1925 98.7291) (end 129.1925 99.6315) (width 0.1524) (layer F.Cu) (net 19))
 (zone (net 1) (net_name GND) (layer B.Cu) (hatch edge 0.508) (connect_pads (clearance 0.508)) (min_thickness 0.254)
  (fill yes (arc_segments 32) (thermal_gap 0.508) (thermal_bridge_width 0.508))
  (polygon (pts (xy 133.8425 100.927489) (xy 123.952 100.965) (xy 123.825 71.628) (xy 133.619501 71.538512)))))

